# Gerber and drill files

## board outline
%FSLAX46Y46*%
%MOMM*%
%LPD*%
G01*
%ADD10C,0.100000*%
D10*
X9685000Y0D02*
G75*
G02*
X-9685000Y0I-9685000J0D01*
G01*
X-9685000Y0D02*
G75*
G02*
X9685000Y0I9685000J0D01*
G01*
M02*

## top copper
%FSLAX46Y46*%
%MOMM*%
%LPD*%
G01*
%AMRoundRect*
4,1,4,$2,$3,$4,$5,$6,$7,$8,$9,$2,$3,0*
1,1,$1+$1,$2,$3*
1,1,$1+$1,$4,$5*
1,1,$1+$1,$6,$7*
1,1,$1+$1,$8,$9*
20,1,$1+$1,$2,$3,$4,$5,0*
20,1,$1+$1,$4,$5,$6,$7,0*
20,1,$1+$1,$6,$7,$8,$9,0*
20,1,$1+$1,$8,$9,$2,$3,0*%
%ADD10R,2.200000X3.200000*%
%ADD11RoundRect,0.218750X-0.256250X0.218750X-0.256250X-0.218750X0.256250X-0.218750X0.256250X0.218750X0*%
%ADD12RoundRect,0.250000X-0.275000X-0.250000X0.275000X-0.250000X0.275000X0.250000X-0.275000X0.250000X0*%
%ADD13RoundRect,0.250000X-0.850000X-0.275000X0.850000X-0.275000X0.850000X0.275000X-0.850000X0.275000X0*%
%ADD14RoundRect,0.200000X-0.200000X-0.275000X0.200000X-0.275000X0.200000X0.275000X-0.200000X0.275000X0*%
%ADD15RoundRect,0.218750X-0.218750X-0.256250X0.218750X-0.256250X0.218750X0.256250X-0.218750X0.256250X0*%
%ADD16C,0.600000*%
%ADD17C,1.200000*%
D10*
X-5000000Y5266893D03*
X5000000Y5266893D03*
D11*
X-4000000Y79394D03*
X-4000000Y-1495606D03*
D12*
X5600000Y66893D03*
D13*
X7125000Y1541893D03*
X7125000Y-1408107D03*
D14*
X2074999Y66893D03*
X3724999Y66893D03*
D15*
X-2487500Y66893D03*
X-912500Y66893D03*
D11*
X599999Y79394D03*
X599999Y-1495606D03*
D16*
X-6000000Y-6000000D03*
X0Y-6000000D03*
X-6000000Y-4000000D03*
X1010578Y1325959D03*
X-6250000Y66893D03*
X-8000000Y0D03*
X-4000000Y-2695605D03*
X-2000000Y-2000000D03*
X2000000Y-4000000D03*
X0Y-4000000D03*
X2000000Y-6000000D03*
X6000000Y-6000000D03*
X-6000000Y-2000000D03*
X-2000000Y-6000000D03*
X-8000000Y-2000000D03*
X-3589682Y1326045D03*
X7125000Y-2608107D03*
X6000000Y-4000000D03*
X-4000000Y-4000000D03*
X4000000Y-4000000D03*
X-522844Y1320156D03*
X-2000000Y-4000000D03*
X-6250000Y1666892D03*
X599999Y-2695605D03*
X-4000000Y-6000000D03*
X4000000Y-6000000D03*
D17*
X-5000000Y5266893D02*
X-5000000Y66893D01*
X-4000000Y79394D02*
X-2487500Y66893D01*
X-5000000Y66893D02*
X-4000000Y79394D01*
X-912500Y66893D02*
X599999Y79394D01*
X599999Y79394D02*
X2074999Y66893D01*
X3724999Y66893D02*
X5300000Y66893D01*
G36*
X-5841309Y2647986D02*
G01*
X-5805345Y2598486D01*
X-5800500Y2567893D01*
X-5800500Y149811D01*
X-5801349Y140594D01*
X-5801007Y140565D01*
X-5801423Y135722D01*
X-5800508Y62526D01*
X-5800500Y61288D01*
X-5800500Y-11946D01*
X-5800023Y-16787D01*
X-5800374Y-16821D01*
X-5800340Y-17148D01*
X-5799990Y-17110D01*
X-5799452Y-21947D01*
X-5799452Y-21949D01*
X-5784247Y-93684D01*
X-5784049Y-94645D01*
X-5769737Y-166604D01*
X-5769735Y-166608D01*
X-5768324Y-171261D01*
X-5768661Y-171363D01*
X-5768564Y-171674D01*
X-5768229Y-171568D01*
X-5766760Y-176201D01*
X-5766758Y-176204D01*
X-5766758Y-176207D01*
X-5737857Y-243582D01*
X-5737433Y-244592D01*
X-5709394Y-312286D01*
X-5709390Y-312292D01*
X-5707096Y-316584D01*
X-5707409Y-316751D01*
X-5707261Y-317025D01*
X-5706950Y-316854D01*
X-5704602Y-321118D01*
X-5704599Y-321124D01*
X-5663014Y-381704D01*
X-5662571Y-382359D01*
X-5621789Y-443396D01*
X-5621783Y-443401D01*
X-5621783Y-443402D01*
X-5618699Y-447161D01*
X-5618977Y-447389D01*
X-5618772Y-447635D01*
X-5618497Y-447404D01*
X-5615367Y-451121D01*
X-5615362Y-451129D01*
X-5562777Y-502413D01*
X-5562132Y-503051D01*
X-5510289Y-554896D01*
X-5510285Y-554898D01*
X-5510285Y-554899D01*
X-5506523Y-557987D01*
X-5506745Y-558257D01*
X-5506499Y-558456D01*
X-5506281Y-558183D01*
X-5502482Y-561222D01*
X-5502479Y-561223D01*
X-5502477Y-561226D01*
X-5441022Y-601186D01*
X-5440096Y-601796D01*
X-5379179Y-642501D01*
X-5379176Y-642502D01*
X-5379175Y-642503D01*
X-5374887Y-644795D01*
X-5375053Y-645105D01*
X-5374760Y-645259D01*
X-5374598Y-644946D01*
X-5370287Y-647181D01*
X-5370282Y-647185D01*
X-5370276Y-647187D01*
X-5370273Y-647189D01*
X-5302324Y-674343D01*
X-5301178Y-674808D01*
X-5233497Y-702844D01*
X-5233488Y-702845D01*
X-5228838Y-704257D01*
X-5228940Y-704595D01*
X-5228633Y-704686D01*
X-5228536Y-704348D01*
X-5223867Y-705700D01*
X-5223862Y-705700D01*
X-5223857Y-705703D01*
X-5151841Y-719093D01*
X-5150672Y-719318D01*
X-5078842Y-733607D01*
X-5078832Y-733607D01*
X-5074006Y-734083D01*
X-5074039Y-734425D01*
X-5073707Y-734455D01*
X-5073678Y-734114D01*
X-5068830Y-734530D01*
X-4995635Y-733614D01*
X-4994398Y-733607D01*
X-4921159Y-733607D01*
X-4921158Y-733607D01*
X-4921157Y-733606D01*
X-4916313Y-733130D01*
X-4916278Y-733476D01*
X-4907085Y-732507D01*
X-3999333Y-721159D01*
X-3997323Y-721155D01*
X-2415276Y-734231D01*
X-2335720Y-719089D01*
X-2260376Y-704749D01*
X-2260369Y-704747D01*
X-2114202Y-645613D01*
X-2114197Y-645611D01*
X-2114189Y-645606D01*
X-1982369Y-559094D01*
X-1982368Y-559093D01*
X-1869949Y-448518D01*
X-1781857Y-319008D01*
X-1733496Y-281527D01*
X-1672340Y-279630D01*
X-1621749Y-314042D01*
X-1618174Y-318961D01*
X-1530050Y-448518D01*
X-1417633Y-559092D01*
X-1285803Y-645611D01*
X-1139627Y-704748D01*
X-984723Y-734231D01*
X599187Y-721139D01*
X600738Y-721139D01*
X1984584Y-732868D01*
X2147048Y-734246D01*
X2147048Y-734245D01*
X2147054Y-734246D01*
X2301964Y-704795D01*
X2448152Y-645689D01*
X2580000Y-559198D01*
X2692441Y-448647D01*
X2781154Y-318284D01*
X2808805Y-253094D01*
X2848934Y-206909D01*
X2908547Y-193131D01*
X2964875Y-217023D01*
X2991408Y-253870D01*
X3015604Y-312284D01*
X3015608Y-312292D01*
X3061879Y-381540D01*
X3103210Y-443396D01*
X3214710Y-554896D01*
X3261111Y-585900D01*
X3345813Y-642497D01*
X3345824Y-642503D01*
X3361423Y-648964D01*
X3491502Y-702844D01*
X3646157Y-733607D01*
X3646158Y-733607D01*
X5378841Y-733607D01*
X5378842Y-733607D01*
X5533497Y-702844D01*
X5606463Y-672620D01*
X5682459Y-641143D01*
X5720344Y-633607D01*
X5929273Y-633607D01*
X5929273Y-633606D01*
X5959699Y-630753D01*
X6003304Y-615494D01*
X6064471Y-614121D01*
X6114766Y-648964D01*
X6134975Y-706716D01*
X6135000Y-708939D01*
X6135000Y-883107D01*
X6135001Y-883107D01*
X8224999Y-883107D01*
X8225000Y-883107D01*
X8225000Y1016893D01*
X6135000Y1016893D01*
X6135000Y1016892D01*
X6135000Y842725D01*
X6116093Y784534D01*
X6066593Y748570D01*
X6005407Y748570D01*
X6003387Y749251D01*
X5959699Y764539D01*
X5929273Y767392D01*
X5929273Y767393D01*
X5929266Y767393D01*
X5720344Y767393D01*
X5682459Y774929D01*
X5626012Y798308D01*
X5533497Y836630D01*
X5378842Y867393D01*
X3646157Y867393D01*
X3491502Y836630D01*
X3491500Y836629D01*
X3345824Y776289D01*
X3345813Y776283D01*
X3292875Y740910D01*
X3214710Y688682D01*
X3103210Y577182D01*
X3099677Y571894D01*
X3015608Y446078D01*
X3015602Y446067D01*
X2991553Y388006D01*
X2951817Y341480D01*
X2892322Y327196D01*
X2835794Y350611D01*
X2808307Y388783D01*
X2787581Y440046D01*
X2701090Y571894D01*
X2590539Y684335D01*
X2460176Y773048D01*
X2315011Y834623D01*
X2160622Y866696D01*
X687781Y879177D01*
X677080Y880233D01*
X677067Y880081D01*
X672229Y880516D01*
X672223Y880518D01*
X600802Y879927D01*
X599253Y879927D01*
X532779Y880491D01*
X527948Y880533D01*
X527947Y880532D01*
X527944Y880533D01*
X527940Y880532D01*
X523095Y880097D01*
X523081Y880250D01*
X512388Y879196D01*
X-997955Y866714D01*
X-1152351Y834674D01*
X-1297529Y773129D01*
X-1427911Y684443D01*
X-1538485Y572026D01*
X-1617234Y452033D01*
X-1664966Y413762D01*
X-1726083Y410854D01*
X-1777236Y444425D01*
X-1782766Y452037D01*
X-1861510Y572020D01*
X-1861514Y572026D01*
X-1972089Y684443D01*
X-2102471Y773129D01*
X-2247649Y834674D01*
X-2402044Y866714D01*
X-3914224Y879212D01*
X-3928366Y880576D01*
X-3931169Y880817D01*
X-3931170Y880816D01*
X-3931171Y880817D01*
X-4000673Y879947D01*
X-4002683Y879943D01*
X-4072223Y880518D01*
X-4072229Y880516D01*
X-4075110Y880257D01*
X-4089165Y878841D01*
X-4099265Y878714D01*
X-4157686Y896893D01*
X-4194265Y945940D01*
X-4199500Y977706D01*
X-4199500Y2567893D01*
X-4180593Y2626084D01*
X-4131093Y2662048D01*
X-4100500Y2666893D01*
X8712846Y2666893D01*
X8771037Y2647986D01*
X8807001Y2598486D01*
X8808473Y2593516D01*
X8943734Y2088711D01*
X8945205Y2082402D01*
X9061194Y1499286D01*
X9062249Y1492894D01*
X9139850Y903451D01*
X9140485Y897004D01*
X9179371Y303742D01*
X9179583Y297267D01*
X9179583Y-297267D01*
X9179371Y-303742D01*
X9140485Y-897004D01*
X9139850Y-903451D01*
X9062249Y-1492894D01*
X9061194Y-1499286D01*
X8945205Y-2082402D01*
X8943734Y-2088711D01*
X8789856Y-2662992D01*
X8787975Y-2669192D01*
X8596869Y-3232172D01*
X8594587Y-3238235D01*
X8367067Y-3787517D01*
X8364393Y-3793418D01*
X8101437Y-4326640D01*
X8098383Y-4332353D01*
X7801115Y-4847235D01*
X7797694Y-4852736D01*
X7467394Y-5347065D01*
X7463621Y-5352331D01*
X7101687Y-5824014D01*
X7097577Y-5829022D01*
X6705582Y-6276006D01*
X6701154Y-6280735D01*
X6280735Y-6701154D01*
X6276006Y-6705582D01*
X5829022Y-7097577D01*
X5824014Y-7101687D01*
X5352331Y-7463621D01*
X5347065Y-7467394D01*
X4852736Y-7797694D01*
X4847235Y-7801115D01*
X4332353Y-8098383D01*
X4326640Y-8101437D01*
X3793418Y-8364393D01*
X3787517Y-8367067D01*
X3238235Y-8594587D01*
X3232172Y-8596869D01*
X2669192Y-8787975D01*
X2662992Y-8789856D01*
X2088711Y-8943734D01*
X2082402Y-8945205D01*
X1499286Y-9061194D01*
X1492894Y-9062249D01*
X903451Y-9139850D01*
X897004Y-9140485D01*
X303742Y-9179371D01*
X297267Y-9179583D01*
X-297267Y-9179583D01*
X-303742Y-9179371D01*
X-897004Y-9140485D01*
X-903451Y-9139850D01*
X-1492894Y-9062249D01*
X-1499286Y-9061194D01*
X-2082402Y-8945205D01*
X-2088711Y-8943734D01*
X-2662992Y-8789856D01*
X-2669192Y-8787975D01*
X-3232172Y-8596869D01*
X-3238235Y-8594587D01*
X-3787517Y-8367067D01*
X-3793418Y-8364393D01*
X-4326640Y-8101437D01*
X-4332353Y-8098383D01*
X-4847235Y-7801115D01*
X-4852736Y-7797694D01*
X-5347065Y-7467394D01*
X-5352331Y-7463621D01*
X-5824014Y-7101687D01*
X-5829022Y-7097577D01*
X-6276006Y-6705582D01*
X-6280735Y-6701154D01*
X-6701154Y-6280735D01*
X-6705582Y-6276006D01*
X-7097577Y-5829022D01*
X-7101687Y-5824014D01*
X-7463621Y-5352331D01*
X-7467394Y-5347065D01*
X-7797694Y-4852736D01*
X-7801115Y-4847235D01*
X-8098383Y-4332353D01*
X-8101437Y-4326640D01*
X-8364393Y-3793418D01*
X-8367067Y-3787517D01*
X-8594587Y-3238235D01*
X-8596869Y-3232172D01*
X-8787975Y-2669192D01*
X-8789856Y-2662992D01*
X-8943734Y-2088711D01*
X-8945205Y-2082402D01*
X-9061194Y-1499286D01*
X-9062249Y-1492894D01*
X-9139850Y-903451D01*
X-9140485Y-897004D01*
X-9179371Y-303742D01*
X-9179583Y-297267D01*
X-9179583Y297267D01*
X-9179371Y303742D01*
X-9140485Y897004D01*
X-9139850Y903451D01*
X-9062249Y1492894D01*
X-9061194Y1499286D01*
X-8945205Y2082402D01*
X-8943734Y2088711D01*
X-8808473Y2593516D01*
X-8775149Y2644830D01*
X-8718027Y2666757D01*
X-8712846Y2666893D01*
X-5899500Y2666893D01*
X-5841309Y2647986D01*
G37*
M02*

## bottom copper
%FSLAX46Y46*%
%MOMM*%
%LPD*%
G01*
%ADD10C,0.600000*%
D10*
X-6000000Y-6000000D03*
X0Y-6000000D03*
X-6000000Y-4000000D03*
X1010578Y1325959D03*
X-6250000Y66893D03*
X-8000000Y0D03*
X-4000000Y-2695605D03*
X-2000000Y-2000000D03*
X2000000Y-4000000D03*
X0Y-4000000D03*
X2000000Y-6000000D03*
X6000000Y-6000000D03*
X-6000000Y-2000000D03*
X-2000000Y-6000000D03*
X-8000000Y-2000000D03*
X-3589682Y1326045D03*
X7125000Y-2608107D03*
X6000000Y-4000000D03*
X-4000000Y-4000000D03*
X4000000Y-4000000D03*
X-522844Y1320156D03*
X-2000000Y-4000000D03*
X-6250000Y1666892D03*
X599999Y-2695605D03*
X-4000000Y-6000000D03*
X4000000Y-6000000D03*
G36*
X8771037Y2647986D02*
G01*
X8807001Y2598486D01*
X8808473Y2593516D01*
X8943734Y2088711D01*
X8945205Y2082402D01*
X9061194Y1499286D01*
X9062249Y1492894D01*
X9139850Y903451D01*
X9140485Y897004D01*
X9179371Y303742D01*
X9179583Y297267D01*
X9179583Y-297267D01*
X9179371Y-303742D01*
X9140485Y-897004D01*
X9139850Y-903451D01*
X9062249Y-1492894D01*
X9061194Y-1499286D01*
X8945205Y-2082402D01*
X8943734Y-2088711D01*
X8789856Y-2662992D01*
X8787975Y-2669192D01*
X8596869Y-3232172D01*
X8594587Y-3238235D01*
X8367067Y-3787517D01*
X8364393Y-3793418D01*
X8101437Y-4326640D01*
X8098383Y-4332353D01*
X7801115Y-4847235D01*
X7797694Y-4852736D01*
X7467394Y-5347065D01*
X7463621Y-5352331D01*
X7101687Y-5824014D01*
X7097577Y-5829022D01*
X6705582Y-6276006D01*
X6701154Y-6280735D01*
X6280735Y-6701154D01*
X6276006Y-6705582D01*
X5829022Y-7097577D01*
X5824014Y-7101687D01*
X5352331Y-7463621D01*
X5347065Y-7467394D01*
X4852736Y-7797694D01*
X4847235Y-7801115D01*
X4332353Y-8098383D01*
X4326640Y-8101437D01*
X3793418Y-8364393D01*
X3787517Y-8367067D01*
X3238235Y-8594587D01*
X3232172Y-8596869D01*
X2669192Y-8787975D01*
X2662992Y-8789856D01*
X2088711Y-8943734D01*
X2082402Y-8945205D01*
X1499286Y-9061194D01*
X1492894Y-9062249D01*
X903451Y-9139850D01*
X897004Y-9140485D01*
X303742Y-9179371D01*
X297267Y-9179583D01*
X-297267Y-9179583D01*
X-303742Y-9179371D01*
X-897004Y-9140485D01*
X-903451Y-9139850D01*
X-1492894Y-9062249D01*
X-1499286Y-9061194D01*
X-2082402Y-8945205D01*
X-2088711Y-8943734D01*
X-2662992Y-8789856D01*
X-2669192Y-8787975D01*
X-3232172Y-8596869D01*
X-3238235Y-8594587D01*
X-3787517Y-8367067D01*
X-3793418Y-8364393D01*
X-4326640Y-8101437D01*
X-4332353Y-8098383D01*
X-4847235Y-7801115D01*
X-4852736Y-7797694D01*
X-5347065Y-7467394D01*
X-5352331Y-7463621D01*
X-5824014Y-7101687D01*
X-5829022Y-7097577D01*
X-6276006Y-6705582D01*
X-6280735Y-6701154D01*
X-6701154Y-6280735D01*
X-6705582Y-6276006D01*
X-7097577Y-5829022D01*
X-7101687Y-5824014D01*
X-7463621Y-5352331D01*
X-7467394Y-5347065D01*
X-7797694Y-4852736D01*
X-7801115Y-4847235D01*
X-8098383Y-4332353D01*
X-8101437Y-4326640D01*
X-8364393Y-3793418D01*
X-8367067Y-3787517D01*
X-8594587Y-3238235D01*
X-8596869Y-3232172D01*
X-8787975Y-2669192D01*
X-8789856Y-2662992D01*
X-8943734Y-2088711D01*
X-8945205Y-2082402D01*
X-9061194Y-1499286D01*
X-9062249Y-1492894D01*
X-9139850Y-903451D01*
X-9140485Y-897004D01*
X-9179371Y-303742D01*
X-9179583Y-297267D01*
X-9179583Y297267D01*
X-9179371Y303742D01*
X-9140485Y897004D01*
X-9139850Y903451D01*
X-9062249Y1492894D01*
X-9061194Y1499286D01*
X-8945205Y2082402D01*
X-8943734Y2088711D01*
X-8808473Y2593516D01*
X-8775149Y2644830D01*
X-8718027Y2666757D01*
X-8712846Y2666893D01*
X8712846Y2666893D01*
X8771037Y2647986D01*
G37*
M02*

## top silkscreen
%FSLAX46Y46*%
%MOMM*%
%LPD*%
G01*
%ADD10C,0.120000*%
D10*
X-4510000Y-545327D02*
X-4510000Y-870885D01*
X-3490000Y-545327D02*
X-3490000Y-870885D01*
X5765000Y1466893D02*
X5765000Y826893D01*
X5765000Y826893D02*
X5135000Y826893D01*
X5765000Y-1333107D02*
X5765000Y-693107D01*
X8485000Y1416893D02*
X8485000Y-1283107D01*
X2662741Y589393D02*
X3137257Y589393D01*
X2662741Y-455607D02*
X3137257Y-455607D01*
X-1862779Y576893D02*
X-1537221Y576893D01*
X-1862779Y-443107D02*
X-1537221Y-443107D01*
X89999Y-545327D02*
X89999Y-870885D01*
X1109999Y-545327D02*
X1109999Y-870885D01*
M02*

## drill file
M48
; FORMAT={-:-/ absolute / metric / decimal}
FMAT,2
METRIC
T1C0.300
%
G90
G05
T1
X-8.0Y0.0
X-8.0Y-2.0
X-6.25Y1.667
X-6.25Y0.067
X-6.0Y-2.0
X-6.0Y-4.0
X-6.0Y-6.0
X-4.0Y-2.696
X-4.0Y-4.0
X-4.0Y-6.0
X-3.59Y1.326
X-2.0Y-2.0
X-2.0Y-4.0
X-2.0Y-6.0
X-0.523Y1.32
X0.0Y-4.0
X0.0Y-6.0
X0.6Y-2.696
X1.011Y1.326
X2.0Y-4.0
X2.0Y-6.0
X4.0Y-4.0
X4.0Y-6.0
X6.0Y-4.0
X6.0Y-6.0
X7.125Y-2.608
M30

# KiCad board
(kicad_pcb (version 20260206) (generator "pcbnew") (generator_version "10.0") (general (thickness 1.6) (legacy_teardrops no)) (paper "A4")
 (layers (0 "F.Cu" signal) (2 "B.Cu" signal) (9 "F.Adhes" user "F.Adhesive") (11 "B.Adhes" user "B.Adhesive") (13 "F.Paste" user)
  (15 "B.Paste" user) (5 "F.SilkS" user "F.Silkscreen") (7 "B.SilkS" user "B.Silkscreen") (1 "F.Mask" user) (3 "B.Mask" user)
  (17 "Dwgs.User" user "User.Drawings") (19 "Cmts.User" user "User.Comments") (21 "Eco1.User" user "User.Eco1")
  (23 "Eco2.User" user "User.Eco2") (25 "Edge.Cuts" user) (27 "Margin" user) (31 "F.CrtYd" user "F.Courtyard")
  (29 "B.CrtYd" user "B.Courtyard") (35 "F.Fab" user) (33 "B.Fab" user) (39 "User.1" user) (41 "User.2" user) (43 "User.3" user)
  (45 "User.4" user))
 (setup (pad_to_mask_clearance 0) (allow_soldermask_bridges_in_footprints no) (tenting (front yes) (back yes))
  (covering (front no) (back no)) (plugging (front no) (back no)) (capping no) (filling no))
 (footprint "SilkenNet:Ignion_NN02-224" (layer "F.Cu") (at 0 -5.266893)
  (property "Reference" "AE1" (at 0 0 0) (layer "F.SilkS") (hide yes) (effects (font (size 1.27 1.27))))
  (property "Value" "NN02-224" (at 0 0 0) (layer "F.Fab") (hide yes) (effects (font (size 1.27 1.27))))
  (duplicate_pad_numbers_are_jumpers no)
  (pad "1" smd rect (at -5 0) (size 2.2 3.2) (layers "F.Cu" "F.Mask" "F.Paste") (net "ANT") (thermal_bridge_angle 45))
  (pad "2" smd rect (at 5 0) (size 2.2 3.2) (layers "F.Cu" "F.Mask" "F.Paste") (thermal_bridge_angle 45)))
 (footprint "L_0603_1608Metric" (layer "F.Cu") (at -4 0.708106 -90)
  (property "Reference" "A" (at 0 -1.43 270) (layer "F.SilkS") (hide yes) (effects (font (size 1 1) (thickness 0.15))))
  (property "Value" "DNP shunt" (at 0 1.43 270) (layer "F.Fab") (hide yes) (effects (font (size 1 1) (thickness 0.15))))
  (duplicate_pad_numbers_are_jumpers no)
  (fp_line (start -0.162779 0.51) (end 0.162779 0.51) (stroke (width 0.12) (type solid)) (layer "F.SilkS"))
  (fp_line (start -0.162779 -0.51) (end 0.162779 -0.51) (stroke (width 0.12) (type solid)) (layer "F.SilkS"))
  (pad "1" smd roundrect (at -0.7875 0 270) (size 0.875 0.95) (layers "F.Cu" "F.Mask" "F.Paste") (roundrect_rratio 0.25) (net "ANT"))
  (pad "2" smd roundrect (at 0.7875 0 270) (size 0.875 0.95) (layers "F.Cu" "F.Mask" "F.Paste") (roundrect_rratio 0.25) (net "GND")))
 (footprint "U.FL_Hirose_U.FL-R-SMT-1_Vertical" (layer "F.Cu") (at 7.125 -0.066893)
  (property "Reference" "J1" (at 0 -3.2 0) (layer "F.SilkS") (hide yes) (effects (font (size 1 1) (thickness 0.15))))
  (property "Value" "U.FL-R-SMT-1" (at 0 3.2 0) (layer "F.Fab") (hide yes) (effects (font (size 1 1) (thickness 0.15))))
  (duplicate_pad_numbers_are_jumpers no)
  (fp_line (start -1.36 -1.4) (end -1.36 -0.76) (stroke (width 0.12) (type solid)) (layer "F.SilkS"))
  (fp_line (start -1.36 -0.76) (end -1.99 -0.76) (stroke (width 0.12) (type solid)) (layer "F.SilkS"))
  (fp_line (start -1.36 1.4) (end -1.36 0.76) (stroke (width 0.12) (type solid)) (layer "F.SilkS"))
  (fp_line (start 1.36 -1.35) (end 1.36 1.35) (stroke (width 0.12) (type solid)) (layer "F.SilkS"))
  (pad "1" smd roundrect (at -1.525 0) (size 1.05 1) (layers "F.Cu" "F.Mask" "F.Paste") (roundrect_rratio 0.25) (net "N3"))
  (pad "2" smd roundrect (at 0 -1.475) (size 2.2 1.05) (layers "F.Cu" "F.Mask" "F.Paste") (roundrect_rratio 0.2380952381) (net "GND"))
  (pad "2" smd roundrect (at 0 1.475) (size 2.2 1.05) (layers "F.Cu" "F.Mask" "F.Paste") (roundrect_rratio 0.2380952381) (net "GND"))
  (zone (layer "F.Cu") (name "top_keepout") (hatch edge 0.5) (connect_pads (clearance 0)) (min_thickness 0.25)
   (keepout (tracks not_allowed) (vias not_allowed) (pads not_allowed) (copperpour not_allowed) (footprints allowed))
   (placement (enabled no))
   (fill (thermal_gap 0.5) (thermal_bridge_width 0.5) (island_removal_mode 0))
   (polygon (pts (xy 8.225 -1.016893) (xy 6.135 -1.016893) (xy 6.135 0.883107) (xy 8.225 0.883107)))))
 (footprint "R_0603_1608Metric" (layer "F.Cu") (at 2.899999 -0.066893)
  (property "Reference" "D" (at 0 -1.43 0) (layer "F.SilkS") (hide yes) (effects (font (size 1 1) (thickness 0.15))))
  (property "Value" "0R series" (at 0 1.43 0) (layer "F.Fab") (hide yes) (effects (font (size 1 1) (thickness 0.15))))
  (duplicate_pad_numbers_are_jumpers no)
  (fp_line (start -0.237258 -0.5225) (end 0.237258 -0.5225) (stroke (width 0.12) (type solid)) (layer "F.SilkS"))
  (fp_line (start -0.237258 0.5225) (end 0.237258 0.5225) (stroke (width 0.12) (type solid)) (layer "F.SilkS"))
  (pad "1" smd roundrect (at -0.825 0) (size 0.8 0.95) (layers "F.Cu" "F.Mask" "F.Paste") (roundrect_rratio 0.25) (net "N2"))
  (pad "2" smd roundrect (at 0.825 0) (size 0.8 0.95) (layers "F.Cu" "F.Mask" "F.Paste") (roundrect_rratio 0.25) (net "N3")))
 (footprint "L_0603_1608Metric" (layer "F.Cu") (at -1.7 -0.066893)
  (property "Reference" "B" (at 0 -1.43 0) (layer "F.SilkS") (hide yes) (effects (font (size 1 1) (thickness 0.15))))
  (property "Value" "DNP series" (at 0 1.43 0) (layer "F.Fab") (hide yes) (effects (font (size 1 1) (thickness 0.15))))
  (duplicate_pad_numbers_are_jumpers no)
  (fp_line (start -0.162779 -0.51) (end 0.162779 -0.51) (stroke (width 0.12) (type solid)) (layer "F.SilkS"))
  (fp_line (start -0.162779 0.51) (end 0.162779 0.51) (stroke (width 0.12) (type solid)) (layer "F.SilkS"))
  (pad "1" smd roundrect (at -0.7875 0) (size 0.875 0.95) (layers "F.Cu" "F.Mask" "F.Paste") (roundrect_rratio 0.25) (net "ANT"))
  (pad "2" smd roundrect (at 0.7875 0) (size 0.875 0.95) (layers "F.Cu" "F.Mask" "F.Paste") (roundrect_rratio 0.25) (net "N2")))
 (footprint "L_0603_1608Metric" (layer "F.Cu") (at 0.599999 0.708106 -90)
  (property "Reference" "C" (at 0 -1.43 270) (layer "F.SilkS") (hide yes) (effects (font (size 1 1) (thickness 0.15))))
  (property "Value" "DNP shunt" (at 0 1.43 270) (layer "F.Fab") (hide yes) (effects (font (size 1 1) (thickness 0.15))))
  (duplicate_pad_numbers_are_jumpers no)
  (fp_line (start -0.162779 0.51) (end 0.162779 0.51) (stroke (width 0.12) (type solid)) (layer "F.SilkS"))
  (fp_line (start -0.162779 -0.51) (end 0.162779 -0.51) (stroke (width 0.12) (type solid)) (layer "F.SilkS"))
  (pad "1" smd roundrect (at -0.7875 0 270) (size 0.875 0.95) (layers "F.Cu" "F.Mask" "F.Paste") (roundrect_rratio 0.25) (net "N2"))
  (pad "2" smd roundrect (at 0.7875 0 270) (size 0.875 0.95) (layers "F.Cu" "F.Mask" "F.Paste") (roundrect_rratio 0.25) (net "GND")))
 (gr_circle (center 0 0) (end 9.685 0) (stroke (width 0.1) (type default)) (fill no) (layer "Edge.Cuts"))
 (via (at -6 6) (size 0.6) (drill 0.3) (layers "F.Cu" "B.Cu") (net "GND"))
 (via (at 0 6) (size 0.6) (drill 0.3) (layers "F.Cu" "B.Cu") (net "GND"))
 (via (at -6 4) (size 0.6) (drill 0.3) (layers "F.Cu" "B.Cu") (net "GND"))
 (via (at 1.010578 -1.325959) (size 0.6) (drill 0.3) (layers "F.Cu" "B.Cu") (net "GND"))
 (via (at -6.25 -0.066893) (size 0.6) (drill 0.3) (layers "F.Cu" "B.Cu") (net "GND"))
 (via (at -8 0) (size 0.6) (drill 0.3) (layers "F.Cu" "B.Cu") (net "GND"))
 (via (at -4 2.695605) (size 0.6) (drill 0.3) (layers "F.Cu" "B.Cu") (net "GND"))
 (via (at -2 2) (size 0.6) (drill 0.3) (layers "F.Cu" "B.Cu") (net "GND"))
 (via (at 2 4) (size 0.6) (drill 0.3) (layers "F.Cu" "B.Cu") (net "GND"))
 (via (at 0 4) (size 0.6) (drill 0.3) (layers "F.Cu" "B.Cu") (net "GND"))
 (via (at 2 6) (size 0.6) (drill 0.3) (layers "F.Cu" "B.Cu") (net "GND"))
 (via (at 6 6) (size 0.6) (drill 0.3) (layers "F.Cu" "B.Cu") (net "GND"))
 (via (at -6 2) (size 0.6) (drill 0.3) (layers "F.Cu" "B.Cu") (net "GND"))
 (via (at -2 6) (size 0.6) (drill 0.3) (layers "F.Cu" "B.Cu") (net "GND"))
 (via (at -8 2) (size 0.6) (drill 0.3) (layers "F.Cu" "B.Cu") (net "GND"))
 (via (at -3.589682 -1.326045) (size 0.6) (drill 0.3) (layers "F.Cu" "B.Cu") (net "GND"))
 (via (at 7.125 2.608107) (size 0.6) (drill 0.3) (layers "F.Cu" "B.Cu") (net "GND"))
 (via (at 6 4) (size 0.6) (drill 0.3) (layers "F.Cu" "B.Cu") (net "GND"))
 (via (at -4 4) (size 0.6) (drill 0.3) (layers "F.Cu" "B.Cu") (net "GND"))
 (via (at 4 4) (size 0.6) (drill 0.3) (layers "F.Cu" "B.Cu") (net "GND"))
 (via (at -0.522844 -1.320156) (size 0.6) (drill 0.3) (layers "F.Cu" "B.Cu") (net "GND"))
 (via (at -2 4) (size 0.6) (drill 0.3) (layers "F.Cu" "B.Cu") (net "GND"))
 (via (at -6.25 -1.666892) (size 0.6) (drill 0.3) (layers "F.Cu" "B.Cu") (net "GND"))
 (via (at 0.599999 2.695605) (size 0.6) (drill 0.3) (layers "F.Cu" "B.Cu") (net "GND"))
 (via (at -4 6) (size 0.6) (drill 0.3) (layers "F.Cu" "B.Cu") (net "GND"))
 (via (at 4 6) (size 0.6) (drill 0.3) (layers "F.Cu" "B.Cu") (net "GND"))
 (segment (start -5 -5.266893) (end -5 -0.066893) (width 1.2) (layer "F.Cu") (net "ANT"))
 (segment (start -4 -0.079394) (end -2.4875 -0.066893) (width 1.2) (layer "F.Cu") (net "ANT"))
 (segment (start -5 -0.066893) (end -4 -0.079394) (width 1.2) (layer "F.Cu") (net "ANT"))
 (segment (start -0.9125 -0.066893) (end 0.599999 -0.079394) (width 1.2) (layer "F.Cu") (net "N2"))
 (segment (start 0.599999 -0.079394) (end 2.074999 -0.066893) (width 1.2) (layer "F.Cu") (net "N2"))
 (segment (start 3.724999 -0.066893) (end 5.3 -0.066893) (width 1.2) (layer "F.Cu") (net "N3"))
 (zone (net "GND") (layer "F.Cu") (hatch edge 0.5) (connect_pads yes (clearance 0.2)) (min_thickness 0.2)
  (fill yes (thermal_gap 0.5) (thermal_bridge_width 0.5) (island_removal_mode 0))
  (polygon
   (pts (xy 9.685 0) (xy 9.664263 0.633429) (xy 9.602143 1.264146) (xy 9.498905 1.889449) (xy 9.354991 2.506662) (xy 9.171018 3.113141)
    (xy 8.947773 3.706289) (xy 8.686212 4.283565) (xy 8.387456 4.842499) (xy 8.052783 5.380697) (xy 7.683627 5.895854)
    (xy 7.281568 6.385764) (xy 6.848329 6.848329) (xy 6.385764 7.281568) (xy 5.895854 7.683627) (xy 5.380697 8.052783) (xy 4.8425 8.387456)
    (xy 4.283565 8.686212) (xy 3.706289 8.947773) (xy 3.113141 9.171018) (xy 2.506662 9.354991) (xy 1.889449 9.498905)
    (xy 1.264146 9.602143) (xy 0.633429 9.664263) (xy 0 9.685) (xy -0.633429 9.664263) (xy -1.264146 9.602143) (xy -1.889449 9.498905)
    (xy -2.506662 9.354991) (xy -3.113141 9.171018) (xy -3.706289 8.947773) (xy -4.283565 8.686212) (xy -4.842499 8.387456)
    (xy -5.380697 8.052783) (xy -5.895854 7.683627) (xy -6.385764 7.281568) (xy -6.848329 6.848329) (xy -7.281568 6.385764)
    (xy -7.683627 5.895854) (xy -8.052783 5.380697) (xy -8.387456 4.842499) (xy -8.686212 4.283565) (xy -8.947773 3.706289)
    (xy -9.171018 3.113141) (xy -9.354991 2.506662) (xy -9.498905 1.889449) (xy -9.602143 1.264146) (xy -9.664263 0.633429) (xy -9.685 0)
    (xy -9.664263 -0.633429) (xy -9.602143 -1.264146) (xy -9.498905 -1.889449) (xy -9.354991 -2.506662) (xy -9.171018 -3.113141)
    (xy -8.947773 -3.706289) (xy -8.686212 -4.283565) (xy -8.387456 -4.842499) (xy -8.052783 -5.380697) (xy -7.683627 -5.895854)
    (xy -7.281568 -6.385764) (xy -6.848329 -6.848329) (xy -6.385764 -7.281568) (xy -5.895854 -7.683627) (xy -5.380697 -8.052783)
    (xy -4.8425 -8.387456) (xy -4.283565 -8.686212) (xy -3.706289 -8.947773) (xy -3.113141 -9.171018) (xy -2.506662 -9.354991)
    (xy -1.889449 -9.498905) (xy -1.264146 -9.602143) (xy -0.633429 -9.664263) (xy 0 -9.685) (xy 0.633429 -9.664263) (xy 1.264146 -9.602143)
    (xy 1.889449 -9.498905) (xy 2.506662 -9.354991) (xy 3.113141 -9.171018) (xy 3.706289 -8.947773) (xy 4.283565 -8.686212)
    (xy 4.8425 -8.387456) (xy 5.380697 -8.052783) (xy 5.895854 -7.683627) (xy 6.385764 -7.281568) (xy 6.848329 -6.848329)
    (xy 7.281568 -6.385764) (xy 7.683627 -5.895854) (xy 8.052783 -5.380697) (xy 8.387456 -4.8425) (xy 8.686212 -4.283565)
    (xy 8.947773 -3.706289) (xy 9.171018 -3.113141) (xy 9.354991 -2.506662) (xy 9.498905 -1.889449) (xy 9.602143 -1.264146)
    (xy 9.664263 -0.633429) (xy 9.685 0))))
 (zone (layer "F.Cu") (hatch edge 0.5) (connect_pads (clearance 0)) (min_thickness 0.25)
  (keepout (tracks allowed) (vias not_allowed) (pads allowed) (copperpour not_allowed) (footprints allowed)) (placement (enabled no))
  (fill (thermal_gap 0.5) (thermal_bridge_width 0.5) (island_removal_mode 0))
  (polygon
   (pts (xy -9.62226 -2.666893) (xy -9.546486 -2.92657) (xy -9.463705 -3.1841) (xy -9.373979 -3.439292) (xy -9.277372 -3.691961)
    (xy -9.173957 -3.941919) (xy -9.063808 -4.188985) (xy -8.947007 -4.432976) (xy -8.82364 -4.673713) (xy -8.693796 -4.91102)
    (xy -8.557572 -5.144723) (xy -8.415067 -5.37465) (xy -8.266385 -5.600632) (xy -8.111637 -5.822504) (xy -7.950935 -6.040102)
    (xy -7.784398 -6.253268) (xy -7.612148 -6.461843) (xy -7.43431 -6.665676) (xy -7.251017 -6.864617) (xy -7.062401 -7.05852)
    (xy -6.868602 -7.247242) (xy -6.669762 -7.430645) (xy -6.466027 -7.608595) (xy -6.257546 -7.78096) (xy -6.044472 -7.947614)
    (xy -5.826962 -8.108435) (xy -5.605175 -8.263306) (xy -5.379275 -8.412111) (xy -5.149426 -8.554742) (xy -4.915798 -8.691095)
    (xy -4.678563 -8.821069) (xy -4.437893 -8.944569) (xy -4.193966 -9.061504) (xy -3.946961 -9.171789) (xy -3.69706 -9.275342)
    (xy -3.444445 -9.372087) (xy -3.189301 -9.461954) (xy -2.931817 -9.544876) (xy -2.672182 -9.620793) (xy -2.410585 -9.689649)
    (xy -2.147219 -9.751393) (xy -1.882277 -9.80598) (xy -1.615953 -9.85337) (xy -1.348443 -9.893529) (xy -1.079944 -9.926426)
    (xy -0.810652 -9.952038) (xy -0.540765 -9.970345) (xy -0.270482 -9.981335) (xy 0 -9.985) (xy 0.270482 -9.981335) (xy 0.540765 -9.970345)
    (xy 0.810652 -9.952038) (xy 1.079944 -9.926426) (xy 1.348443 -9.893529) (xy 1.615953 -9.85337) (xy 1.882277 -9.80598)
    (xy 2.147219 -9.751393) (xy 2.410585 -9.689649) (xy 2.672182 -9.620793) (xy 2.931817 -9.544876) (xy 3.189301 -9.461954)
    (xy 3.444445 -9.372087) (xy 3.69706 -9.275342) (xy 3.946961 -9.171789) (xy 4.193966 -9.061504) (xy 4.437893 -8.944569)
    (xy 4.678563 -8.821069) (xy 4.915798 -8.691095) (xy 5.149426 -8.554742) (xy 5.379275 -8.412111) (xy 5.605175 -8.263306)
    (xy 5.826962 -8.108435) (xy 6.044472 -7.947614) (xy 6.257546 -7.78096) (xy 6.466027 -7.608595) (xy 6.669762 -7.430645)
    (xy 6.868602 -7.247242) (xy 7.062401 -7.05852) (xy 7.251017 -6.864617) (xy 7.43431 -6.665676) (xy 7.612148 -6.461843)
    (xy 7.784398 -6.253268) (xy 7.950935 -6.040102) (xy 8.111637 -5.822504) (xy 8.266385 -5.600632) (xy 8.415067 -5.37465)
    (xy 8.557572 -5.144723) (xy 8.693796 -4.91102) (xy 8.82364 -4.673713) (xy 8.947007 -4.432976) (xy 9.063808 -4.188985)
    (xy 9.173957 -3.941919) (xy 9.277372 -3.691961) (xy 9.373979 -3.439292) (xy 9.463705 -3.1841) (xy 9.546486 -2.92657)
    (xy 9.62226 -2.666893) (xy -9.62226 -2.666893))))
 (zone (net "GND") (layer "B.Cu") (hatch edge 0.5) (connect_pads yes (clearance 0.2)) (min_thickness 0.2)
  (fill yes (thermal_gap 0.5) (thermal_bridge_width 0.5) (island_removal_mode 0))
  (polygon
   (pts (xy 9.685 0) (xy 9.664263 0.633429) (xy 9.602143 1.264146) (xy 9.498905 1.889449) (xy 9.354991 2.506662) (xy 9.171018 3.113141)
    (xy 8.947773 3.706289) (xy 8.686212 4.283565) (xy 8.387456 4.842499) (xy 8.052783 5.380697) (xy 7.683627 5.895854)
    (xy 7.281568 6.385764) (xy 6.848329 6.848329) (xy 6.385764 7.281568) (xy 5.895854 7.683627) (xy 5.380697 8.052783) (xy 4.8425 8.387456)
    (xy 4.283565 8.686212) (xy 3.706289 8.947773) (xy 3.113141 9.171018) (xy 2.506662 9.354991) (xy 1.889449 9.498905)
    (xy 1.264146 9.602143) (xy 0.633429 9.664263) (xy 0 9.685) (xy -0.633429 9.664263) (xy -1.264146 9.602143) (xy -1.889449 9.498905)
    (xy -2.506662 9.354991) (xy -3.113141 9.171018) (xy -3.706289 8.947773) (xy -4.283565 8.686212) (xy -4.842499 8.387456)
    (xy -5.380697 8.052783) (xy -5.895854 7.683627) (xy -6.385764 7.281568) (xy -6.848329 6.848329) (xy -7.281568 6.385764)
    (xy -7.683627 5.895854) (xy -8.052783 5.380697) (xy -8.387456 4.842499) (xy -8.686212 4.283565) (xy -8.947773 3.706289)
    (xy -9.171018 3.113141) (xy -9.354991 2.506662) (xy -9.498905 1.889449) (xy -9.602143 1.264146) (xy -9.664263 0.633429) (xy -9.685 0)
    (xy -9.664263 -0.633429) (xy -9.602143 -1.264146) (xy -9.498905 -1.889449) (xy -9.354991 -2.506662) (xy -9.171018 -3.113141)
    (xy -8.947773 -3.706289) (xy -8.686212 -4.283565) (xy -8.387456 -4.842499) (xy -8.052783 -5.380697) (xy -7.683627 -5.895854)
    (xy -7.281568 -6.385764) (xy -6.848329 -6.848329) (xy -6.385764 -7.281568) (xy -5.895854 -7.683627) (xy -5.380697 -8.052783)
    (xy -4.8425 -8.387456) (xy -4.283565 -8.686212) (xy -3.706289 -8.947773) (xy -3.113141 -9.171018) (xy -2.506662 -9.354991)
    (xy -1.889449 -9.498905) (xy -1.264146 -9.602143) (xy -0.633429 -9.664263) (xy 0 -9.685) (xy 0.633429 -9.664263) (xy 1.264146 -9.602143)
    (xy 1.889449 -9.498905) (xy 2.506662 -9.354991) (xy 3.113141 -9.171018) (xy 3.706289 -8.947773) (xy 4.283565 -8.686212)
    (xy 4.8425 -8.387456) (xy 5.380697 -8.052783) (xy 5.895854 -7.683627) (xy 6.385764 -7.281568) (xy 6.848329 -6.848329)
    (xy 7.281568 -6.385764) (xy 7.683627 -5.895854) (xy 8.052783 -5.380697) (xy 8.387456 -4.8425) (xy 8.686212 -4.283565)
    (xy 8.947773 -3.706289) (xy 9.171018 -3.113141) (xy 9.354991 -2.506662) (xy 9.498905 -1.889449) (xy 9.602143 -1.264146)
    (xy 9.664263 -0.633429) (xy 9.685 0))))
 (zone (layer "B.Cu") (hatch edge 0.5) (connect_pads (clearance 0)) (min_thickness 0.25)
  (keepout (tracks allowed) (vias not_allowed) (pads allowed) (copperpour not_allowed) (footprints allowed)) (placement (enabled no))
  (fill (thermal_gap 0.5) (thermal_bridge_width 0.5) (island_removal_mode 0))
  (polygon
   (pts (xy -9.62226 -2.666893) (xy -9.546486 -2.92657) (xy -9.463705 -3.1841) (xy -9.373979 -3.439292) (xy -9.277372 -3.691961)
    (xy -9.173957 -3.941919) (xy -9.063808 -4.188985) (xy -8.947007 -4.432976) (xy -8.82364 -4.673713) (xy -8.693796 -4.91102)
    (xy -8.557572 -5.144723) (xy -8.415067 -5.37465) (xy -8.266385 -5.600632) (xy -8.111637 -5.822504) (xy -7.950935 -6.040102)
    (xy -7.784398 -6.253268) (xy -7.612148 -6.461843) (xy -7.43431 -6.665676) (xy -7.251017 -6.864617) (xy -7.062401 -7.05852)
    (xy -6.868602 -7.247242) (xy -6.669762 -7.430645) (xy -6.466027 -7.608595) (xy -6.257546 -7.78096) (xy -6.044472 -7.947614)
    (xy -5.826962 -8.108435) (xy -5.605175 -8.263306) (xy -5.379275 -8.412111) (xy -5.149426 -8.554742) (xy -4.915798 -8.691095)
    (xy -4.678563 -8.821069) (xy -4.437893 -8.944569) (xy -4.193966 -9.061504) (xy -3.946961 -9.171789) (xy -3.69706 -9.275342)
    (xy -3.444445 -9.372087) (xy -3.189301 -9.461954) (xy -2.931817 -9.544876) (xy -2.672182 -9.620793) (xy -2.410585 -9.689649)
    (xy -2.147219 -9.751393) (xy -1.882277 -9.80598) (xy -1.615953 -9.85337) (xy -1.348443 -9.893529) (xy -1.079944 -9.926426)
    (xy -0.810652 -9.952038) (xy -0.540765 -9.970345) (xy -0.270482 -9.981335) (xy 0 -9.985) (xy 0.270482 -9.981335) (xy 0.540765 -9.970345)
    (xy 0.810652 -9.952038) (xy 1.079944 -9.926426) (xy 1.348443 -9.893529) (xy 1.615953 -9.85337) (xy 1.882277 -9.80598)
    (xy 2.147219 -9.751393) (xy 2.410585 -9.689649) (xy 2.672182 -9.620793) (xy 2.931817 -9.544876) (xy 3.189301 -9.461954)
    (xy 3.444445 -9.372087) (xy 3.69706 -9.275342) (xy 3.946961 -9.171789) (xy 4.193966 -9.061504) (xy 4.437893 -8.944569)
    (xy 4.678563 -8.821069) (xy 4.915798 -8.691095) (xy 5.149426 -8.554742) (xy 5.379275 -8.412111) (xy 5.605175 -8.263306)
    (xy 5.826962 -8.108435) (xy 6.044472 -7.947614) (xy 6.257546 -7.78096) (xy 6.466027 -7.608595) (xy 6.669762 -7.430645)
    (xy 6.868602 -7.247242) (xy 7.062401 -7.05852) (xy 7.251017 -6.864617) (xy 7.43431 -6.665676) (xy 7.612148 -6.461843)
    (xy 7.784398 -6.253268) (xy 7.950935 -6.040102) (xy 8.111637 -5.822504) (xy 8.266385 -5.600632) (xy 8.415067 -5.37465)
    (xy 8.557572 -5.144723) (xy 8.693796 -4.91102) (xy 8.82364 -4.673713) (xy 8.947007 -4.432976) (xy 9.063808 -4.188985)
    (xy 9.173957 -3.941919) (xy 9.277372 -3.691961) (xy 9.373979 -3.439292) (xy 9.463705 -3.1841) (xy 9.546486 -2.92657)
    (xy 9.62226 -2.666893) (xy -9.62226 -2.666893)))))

